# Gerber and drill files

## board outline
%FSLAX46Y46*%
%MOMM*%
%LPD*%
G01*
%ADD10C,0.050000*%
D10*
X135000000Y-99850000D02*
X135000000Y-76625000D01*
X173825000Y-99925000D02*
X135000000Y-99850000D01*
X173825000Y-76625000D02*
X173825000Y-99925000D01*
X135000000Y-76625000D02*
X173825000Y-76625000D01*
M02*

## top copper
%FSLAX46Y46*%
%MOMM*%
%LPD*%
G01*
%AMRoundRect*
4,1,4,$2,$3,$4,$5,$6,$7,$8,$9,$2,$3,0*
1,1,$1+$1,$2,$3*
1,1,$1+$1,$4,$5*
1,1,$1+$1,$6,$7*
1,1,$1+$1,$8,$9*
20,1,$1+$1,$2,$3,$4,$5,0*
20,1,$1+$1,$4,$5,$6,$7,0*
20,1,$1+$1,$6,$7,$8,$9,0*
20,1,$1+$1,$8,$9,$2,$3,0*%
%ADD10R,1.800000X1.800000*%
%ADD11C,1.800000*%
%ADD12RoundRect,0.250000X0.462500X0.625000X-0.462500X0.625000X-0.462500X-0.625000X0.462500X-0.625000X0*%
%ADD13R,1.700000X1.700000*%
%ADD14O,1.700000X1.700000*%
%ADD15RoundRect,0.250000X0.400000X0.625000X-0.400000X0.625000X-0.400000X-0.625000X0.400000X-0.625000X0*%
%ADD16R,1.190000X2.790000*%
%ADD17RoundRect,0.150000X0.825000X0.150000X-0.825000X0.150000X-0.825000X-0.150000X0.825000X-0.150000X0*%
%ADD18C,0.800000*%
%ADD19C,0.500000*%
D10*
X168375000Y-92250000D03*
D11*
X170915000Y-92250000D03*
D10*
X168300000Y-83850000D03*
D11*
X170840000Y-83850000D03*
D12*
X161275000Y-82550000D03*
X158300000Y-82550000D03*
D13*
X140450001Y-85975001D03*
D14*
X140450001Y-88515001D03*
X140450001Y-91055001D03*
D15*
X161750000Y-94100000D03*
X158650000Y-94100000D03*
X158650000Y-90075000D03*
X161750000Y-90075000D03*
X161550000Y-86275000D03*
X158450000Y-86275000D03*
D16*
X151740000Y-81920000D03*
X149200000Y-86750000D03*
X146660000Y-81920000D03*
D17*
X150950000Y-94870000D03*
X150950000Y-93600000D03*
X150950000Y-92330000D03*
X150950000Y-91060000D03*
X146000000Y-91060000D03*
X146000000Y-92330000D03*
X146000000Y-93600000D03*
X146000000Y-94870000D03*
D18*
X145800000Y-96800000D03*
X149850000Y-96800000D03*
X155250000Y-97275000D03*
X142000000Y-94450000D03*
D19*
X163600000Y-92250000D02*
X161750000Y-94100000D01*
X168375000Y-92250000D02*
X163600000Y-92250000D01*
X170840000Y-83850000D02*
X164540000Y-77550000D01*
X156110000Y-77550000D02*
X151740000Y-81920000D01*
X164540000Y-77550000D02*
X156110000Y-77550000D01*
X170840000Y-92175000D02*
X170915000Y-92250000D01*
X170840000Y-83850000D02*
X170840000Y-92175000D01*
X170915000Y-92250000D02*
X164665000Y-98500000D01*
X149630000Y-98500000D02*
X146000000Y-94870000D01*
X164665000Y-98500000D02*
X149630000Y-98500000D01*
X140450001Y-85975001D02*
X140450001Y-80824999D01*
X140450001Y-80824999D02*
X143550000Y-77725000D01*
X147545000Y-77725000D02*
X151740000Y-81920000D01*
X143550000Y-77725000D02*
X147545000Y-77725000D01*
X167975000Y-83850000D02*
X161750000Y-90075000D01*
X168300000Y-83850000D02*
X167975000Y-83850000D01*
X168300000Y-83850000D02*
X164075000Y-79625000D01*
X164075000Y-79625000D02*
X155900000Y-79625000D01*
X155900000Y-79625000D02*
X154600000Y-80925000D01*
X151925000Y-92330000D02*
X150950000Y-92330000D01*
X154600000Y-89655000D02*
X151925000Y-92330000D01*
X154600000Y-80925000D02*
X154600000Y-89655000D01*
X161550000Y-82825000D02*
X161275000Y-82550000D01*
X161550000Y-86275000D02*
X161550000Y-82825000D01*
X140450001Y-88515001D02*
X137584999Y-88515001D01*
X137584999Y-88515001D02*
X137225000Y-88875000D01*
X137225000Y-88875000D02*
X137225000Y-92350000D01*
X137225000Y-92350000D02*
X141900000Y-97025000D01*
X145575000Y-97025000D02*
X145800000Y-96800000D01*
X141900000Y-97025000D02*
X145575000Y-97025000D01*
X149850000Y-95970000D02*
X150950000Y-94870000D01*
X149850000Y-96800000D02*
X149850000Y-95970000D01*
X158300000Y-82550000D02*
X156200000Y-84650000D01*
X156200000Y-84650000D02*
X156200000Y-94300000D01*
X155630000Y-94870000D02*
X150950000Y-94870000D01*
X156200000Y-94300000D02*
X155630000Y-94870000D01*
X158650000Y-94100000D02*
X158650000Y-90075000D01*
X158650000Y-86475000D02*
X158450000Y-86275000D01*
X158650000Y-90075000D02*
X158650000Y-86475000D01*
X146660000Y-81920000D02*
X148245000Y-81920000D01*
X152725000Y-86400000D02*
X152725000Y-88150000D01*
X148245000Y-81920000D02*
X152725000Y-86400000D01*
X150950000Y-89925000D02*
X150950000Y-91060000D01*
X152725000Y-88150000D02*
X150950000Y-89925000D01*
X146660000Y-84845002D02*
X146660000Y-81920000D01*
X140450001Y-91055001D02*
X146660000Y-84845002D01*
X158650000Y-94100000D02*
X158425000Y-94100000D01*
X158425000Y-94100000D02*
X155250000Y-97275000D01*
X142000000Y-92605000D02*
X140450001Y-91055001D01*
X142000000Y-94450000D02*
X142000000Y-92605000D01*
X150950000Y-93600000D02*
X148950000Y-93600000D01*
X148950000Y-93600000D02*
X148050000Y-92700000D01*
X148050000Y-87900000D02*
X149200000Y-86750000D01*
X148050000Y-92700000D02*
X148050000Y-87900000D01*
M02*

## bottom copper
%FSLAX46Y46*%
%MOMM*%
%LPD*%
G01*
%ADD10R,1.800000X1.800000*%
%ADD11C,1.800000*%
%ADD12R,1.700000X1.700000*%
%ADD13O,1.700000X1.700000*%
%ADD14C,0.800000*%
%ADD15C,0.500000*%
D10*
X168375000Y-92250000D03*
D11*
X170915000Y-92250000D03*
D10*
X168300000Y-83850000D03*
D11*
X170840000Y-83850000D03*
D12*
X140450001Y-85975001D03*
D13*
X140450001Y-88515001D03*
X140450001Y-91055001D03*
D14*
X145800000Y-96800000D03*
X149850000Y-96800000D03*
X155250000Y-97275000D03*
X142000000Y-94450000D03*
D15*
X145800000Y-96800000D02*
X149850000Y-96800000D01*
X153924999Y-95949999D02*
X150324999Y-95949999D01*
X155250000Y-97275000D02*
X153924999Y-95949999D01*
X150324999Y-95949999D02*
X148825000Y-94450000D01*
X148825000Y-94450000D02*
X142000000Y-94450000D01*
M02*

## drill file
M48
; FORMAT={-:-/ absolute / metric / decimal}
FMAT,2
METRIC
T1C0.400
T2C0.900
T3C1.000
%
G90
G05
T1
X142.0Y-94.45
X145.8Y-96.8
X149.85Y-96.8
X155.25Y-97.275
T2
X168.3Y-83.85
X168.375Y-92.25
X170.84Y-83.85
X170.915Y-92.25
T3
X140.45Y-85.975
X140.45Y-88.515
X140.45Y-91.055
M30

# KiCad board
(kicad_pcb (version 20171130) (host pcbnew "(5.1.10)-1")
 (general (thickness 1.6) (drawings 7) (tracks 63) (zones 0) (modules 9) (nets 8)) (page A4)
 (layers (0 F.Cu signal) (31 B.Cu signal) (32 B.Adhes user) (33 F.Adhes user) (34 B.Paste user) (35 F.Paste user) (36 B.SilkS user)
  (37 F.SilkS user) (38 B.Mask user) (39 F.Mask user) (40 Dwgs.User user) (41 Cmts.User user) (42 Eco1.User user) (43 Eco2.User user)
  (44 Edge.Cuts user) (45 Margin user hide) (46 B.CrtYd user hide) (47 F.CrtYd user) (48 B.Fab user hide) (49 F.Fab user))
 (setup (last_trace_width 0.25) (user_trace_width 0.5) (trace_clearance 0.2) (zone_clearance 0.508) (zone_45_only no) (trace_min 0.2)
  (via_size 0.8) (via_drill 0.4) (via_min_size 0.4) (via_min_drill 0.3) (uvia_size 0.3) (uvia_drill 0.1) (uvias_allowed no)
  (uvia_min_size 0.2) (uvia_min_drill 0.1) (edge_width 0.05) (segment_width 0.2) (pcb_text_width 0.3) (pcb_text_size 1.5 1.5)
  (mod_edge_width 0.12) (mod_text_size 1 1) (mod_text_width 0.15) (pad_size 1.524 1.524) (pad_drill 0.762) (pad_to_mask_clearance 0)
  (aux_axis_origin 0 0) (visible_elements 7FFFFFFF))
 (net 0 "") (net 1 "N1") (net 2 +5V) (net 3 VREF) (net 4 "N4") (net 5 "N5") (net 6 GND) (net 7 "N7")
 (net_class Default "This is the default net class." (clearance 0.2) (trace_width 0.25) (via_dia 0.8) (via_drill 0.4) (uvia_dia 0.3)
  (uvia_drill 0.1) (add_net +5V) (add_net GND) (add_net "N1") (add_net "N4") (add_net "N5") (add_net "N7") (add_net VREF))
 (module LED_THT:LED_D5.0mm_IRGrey (layer F.Cu) (at 168.375 92.25)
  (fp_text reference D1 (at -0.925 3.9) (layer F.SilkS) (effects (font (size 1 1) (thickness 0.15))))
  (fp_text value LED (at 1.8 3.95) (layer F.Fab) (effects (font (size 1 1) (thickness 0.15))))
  (pad 1 thru_hole rect (at 0 0) (size 1.8 1.8) (drill 0.9) (layers *.Cu *.Mask) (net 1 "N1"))
  (pad 2 thru_hole circle (at 2.54 0) (size 1.8 1.8) (drill 0.9) (layers *.Cu *.Mask) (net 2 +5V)))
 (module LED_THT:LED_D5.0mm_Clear (layer F.Cu) (at 168.3 83.85)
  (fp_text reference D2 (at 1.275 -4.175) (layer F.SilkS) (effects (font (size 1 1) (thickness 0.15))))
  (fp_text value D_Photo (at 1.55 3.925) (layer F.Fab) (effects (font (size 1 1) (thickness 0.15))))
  (pad 1 thru_hole rect (at 0 0) (size 1.8 1.8) (drill 0.9) (layers *.Cu *.Mask) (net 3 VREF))
  (pad 2 thru_hole circle (at 2.54 0) (size 1.8 1.8) (drill 0.9) (layers *.Cu *.Mask) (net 2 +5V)))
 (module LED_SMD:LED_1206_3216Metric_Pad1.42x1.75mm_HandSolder (layer F.Cu) (at 159.7875 82.55 180)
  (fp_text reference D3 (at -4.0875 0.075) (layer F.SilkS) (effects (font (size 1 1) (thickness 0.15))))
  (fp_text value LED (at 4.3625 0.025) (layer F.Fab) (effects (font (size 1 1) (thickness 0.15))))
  (pad 1 smd roundrect (at -1.4875 0 180) (size 1.425 1.75) (layers F.Cu F.Paste F.Mask) (roundrect_rratio 0.1754385964912281) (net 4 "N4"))
  (pad 2 smd roundrect (at 1.4875 0 180) (size 1.425 1.75) (layers F.Cu F.Paste F.Mask) (roundrect_rratio 0.1754385964912281) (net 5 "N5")))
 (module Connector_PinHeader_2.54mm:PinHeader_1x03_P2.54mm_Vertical (layer F.Cu) (at 140.450001 85.975001)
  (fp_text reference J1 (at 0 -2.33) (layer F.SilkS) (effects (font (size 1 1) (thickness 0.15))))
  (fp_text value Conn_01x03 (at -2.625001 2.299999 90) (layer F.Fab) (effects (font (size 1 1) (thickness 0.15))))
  (pad 1 thru_hole rect (at 0 0) (size 1.7 1.7) (drill 1) (layers *.Cu *.Mask) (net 2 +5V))
  (pad 2 thru_hole oval (at 0 2.54) (size 1.7 1.7) (drill 1) (layers *.Cu *.Mask) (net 5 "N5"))
  (pad 3 thru_hole oval (at 0 5.08) (size 1.7 1.7) (drill 1) (layers *.Cu *.Mask) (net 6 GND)))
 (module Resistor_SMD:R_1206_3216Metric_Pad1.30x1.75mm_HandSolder (layer F.Cu) (at 160.2 94.1 180)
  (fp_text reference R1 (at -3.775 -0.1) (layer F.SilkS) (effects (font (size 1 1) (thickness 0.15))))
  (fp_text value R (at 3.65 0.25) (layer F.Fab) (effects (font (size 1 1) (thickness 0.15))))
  (pad 1 smd roundrect (at -1.55 0 180) (size 1.3 1.75) (layers F.Cu F.Paste F.Mask) (roundrect_rratio 0.1923076923076923) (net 1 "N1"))
  (pad 2 smd roundrect (at 1.55 0 180) (size 1.3 1.75) (layers F.Cu F.Paste F.Mask) (roundrect_rratio 0.1923076923076923) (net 6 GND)))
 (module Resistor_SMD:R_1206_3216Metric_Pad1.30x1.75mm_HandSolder (layer F.Cu) (at 160.2 90.075 180)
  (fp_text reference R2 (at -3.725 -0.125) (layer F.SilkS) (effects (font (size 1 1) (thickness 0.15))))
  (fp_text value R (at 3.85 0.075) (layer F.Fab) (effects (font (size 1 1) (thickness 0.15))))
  (pad 2 smd roundrect (at 1.55 0 180) (size 1.3 1.75) (layers F.Cu F.Paste F.Mask) (roundrect_rratio 0.1923076923076923) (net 6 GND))
  (pad 1 smd roundrect (at -1.55 0 180) (size 1.3 1.75) (layers F.Cu F.Paste F.Mask) (roundrect_rratio 0.1923076923076923) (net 3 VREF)))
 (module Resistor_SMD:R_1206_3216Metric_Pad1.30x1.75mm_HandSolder (layer F.Cu) (at 160 86.275 180)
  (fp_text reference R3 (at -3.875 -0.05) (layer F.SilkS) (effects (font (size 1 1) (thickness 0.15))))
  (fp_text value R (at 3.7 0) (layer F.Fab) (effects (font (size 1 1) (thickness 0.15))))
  (pad 1 smd roundrect (at -1.55 0 180) (size 1.3 1.75) (layers F.Cu F.Paste F.Mask) (roundrect_rratio 0.1923076923076923) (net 4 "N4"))
  (pad 2 smd roundrect (at 1.55 0 180) (size 1.3 1.75) (layers F.Cu F.Paste F.Mask) (roundrect_rratio 0.1923076923076923) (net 6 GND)))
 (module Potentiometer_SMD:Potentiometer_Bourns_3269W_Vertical (layer F.Cu) (at 149.2 84.335)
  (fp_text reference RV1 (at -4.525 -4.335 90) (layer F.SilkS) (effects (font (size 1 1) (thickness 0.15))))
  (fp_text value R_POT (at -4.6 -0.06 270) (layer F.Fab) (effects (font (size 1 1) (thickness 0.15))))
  (pad 1 smd rect (at 2.54 -2.415) (size 1.19 2.79) (layers F.Cu F.Paste F.Mask) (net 2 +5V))
  (pad 2 smd rect (at 0 2.415) (size 1.19 2.79) (layers F.Cu F.Paste F.Mask) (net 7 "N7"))
  (pad 3 smd rect (at -2.54 -2.415) (size 1.19 2.79) (layers F.Cu F.Paste F.Mask) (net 6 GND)))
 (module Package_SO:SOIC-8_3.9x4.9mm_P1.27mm (layer F.Cu) (at 148.475 92.965 180)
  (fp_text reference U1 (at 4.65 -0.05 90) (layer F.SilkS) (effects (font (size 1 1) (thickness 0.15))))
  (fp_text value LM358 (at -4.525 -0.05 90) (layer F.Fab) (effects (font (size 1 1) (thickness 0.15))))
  (pad 1 smd roundrect (at -2.475 -1.905 180) (size 1.95 0.6) (layers F.Cu F.Paste F.Mask) (roundrect_rratio 0.25) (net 5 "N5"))
  (pad 2 smd roundrect (at -2.475 -0.635 180) (size 1.95 0.6) (layers F.Cu F.Paste F.Mask) (roundrect_rratio 0.25) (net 7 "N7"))
  (pad 3 smd roundrect (at -2.475 0.635 180) (size 1.95 0.6) (layers F.Cu F.Paste F.Mask) (roundrect_rratio 0.25) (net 3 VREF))
  (pad 4 smd roundrect (at -2.475 1.905 180) (size 1.95 0.6) (layers F.Cu F.Paste F.Mask) (roundrect_rratio 0.25) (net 6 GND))
  (pad 5 smd roundrect (at 2.475 1.905 180) (size 1.95 0.6) (layers F.Cu F.Paste F.Mask) (roundrect_rratio 0.25))
  (pad 6 smd roundrect (at 2.475 0.635 180) (size 1.95 0.6) (layers F.Cu F.Paste F.Mask) (roundrect_rratio 0.25))
  (pad 7 smd roundrect (at 2.475 -0.635 180) (size 1.95 0.6) (layers F.Cu F.Paste F.Mask) (roundrect_rratio 0.25))
  (pad 8 smd roundrect (at 2.475 -1.905 180) (size 1.95 0.6) (layers F.Cu F.Paste F.Mask) (roundrect_rratio 0.25) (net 2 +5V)))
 (gr_line (start 135 99.85) (end 135 76.625) (layer Edge.Cuts) (width 0.05))
 (gr_line (start 173.825 99.925) (end 135 99.85) (layer Edge.Cuts) (width 0.05))
 (gr_line (start 173.825 76.625) (end 173.825 99.925) (layer Edge.Cuts) (width 0.05))
 (gr_line (start 135 76.625) (end 173.825 76.625) (layer Edge.Cuts) (width 0.05))
 (segment (start 163.6 92.25) (end 161.75 94.1) (width 0.5) (layer F.Cu) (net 1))
 (segment (start 168.375 92.25) (end 163.6 92.25) (width 0.5) (layer F.Cu) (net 1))
 (segment (start 170.84 83.85) (end 164.54 77.55) (width 0.5) (layer F.Cu) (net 2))
 (segment (start 156.11 77.55) (end 151.74 81.92) (width 0.5) (layer F.Cu) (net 2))
 (segment (start 164.54 77.55) (end 156.11 77.55) (width 0.5) (layer F.Cu) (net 2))
 (segment (start 170.84 92.175) (end 170.915 92.25) (width 0.5) (layer F.Cu) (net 2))
 (segment (start 170.84 83.85) (end 170.84 92.175) (width 0.5) (layer F.Cu) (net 2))
 (segment (start 170.915 92.25) (end 164.665 98.5) (width 0.5) (layer F.Cu) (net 2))
 (segment (start 149.63 98.5) (end 146 94.87) (width 0.5) (layer F.Cu) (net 2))
 (segment (start 164.665 98.5) (end 149.63 98.5) (width 0.5) (layer F.Cu) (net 2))
 (segment (start 140.450001 85.975001) (end 140.450001 80.824999) (width 0.5) (layer F.Cu) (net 2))
 (segment (start 140.450001 80.824999) (end 143.55 77.725) (width 0.5) (layer F.Cu) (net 2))
 (segment (start 147.545 77.725) (end 151.74 81.92) (width 0.5) (layer F.Cu) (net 2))
 (segment (start 143.55 77.725) (end 147.545 77.725) (width 0.5) (layer F.Cu) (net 2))
 (segment (start 167.975 83.85) (end 161.75 90.075) (width 0.5) (layer F.Cu) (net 3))
 (segment (start 168.3 83.85) (end 167.975 83.85) (width 0.5) (layer F.Cu) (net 3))
 (segment (start 168.3 83.85) (end 164.075 79.625) (width 0.5) (layer F.Cu) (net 3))
 (segment (start 164.075 79.625) (end 155.9 79.625) (width 0.5) (layer F.Cu) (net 3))
 (segment (start 155.9 79.625) (end 154.6 80.925) (width 0.5) (layer F.Cu) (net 3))
 (segment (start 151.925 92.33) (end 150.95 92.33) (width 0.5) (layer F.Cu) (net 3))
 (segment (start 154.6 89.655) (end 151.925 92.33) (width 0.5) (layer F.Cu) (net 3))
 (segment (start 154.6 80.925) (end 154.6 89.655) (width 0.5) (layer F.Cu) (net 3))
 (segment (start 161.55 82.825) (end 161.275 82.55) (width 0.5) (layer F.Cu) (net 4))
 (segment (start 161.55 86.275) (end 161.55 82.825) (width 0.5) (layer F.Cu) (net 4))
 (segment (start 140.450001 88.515001) (end 137.584999 88.515001) (width 0.5) (layer F.Cu) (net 5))
 (segment (start 137.584999 88.515001) (end 137.225 88.875) (width 0.5) (layer F.Cu) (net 5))
 (segment (start 137.225 88.875) (end 137.225 92.35) (width 0.5) (layer F.Cu) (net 5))
 (segment (start 137.225 92.35) (end 141.9 97.025) (width 0.5) (layer F.Cu) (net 5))
 (via (at 145.8 96.8) (size 0.8) (drill 0.4) (layers F.Cu B.Cu) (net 5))
 (segment (start 145.575 97.025) (end 145.8 96.8) (width 0.5) (layer F.Cu) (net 5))
 (segment (start 141.9 97.025) (end 145.575 97.025) (width 0.5) (layer F.Cu) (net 5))
 (segment (start 145.8 96.8) (end 149.85 96.8) (width 0.5) (layer B.Cu) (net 5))
 (via (at 149.85 96.8) (size 0.8) (drill 0.4) (layers F.Cu B.Cu) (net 5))
 (segment (start 149.85 95.97) (end 150.95 94.87) (width 0.5) (layer F.Cu) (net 5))
 (segment (start 149.85 96.8) (end 149.85 95.97) (width 0.5) (layer F.Cu) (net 5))
 (segment (start 158.3 82.55) (end 156.2 84.65) (width 0.5) (layer F.Cu) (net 5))
 (segment (start 156.2 84.65) (end 156.2 94.3) (width 0.5) (layer F.Cu) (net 5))
 (segment (start 155.63 94.87) (end 150.95 94.87) (width 0.5) (layer F.Cu) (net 5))
 (segment (start 156.2 94.3) (end 155.63 94.87) (width 0.5) (layer F.Cu) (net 5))
 (segment (start 158.65 94.1) (end 158.65 90.075) (width 0.5) (layer F.Cu) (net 6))
 (segment (start 158.65 86.475) (end 158.45 86.275) (width 0.5) (layer F.Cu) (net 6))
 (segment (start 158.65 90.075) (end 158.65 86.475) (width 0.5) (layer F.Cu) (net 6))
 (segment (start 146.66 81.92) (end 148.245 81.92) (width 0.5) (layer F.Cu) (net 6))
 (segment (start 152.725 86.4) (end 152.725 88.15) (width 0.5) (layer F.Cu) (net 6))
 (segment (start 148.245 81.92) (end 152.725 86.4) (width 0.5) (layer F.Cu) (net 6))
 (segment (start 150.95 89.925) (end 150.95 91.06) (width 0.5) (layer F.Cu) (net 6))
 (segment (start 152.725 88.15) (end 150.95 89.925) (width 0.5) (layer F.Cu) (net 6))
 (segment (start 146.66 84.845002) (end 146.66 81.92) (width 0.5) (layer F.Cu) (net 6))
 (segment (start 140.450001 91.055001) (end 146.66 84.845002) (width 0.5) (layer F.Cu) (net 6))
 (segment (start 158.65 94.1) (end 158.425 94.1) (width 0.5) (layer F.Cu) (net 6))
 (segment (start 158.425 94.1) (end 155.25 97.275) (width 0.5) (layer F.Cu) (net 6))
 (via (at 155.25 97.275) (size 0.8) (drill 0.4) (layers F.Cu B.Cu) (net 6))
 (segment (start 153.924999 95.949999) (end 150.324999 95.949999) (width 0.5) (layer B.Cu) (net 6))
 (segment (start 155.25 97.275) (end 153.924999 95.949999) (width 0.5) (layer B.Cu) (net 6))
 (segment (start 150.324999 95.949999) (end 148.825 94.45) (width 0.5) (layer B.Cu) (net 6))
 (segment (start 148.825 94.45) (end 142 94.45) (width 0.5) (layer B.Cu) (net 6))
 (via (at 142 94.45) (size 0.8) (drill 0.4) (layers F.Cu B.Cu) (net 6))
 (segment (start 142 92.605) (end 140.450001 91.055001) (width 0.5) (layer F.Cu) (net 6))
 (segment (start 142 94.45) (end 142 92.605) (width 0.5) (layer F.Cu) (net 6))
 (segment (start 150.95 93.6) (end 148.95 93.6) (width 0.5) (layer F.Cu) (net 7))
 (segment (start 148.95 93.6) (end 148.05 92.7) (width 0.5) (layer F.Cu) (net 7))
 (segment (start 148.05 87.9) (end 149.2 86.75) (width 0.5) (layer F.Cu) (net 7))
 (segment (start 148.05 92.7) (end 148.05 87.9) (width 0.5) (layer F.Cu) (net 7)))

